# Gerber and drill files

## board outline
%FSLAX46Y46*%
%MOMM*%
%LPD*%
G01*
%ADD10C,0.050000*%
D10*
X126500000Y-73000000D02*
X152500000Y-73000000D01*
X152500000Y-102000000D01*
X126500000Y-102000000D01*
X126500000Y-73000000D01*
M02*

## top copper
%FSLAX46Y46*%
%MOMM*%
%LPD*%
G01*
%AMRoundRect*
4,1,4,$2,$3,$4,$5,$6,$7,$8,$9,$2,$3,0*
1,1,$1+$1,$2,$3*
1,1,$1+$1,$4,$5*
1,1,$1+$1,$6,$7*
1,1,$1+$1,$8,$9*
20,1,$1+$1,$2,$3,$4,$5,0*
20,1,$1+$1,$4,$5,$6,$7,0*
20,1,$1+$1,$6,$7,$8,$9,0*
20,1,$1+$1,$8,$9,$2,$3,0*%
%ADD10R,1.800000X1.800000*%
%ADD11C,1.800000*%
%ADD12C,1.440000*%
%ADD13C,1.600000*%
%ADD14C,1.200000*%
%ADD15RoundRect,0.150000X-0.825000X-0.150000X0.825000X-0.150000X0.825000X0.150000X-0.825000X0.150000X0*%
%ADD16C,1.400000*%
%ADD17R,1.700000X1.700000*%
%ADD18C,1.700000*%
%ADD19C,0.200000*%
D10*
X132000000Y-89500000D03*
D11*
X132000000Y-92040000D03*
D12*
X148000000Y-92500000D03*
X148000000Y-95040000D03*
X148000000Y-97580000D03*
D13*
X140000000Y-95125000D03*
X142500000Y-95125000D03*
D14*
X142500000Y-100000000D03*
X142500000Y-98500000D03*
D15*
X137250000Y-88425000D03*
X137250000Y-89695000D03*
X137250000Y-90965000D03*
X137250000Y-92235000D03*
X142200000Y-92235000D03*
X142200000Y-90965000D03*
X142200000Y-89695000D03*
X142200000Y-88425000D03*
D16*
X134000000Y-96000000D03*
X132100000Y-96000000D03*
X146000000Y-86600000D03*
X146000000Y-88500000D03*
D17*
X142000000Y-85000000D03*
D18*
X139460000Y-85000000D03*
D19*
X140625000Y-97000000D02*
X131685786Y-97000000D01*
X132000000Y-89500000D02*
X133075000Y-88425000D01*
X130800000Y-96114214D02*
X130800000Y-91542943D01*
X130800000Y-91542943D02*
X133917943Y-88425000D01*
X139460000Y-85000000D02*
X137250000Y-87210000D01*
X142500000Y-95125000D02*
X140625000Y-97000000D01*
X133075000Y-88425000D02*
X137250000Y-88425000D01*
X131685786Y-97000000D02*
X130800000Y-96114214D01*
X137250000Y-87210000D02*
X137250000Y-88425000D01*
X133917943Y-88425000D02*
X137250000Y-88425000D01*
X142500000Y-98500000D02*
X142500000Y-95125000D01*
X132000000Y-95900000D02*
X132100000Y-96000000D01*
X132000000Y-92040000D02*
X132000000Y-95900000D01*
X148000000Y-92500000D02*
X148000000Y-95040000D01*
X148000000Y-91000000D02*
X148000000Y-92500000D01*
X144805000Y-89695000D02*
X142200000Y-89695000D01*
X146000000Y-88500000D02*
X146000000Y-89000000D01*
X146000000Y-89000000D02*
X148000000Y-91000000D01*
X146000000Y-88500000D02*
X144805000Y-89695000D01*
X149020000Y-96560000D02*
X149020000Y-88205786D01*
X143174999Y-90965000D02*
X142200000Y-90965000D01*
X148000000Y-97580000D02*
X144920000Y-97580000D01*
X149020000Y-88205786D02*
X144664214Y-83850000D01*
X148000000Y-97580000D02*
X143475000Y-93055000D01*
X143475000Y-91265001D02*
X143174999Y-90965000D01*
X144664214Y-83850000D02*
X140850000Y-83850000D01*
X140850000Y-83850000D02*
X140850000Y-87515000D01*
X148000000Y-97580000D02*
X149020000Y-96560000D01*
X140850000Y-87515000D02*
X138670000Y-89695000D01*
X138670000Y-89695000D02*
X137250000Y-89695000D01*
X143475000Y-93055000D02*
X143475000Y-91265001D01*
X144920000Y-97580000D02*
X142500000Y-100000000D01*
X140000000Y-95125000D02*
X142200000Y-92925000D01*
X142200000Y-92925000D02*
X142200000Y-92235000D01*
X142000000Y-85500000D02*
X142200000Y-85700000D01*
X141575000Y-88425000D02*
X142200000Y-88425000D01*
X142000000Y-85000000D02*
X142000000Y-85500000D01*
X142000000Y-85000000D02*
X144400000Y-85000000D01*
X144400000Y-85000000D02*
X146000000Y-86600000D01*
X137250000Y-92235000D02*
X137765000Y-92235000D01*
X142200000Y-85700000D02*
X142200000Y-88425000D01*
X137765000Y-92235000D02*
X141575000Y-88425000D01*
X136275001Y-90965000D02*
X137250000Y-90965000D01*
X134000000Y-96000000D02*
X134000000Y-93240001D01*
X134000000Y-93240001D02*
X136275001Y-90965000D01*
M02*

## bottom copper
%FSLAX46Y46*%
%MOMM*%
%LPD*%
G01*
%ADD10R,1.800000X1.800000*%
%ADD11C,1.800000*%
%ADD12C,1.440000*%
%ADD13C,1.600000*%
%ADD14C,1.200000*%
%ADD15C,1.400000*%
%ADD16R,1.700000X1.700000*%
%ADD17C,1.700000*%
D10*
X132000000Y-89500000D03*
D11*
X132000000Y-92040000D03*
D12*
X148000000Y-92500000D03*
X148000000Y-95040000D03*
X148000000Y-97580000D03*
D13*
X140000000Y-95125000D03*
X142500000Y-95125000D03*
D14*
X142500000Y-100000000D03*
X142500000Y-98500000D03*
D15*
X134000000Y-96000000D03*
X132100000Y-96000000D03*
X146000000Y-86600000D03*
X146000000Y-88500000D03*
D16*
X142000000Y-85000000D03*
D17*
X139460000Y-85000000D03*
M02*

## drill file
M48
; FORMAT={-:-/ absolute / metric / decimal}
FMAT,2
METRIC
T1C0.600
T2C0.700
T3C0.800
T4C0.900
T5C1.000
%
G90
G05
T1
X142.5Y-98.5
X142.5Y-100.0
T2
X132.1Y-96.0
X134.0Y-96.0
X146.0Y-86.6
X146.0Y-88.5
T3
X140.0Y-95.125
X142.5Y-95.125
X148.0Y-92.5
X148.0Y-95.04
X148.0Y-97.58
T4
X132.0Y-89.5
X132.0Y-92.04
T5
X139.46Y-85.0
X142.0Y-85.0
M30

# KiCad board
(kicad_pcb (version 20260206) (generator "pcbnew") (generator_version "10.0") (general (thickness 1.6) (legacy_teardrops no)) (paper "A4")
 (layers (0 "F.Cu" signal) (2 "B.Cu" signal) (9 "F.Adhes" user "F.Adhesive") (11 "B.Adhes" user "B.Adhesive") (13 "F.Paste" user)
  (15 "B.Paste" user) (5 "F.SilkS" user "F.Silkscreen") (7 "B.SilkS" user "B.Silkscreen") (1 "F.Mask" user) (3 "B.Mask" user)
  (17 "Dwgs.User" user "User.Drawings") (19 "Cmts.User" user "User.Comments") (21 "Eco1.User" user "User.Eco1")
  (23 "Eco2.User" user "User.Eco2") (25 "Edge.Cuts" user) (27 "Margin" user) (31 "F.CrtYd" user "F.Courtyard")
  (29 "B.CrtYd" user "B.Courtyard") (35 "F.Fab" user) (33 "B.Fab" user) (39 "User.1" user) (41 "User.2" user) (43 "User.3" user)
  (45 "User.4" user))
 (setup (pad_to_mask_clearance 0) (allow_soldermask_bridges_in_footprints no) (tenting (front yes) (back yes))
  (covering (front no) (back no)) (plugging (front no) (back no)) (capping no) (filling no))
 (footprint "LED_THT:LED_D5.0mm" (layer "F.Cu") (at 132 89.5 -90)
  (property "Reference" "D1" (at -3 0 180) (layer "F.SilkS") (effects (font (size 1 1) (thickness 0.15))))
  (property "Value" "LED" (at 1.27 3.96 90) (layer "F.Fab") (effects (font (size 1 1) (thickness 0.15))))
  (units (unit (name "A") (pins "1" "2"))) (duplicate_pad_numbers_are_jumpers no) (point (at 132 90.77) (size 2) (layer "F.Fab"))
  (pad "1" thru_hole rect (at 0 0 270) (size 1.8 1.8) (drill 0.9) (layers "*.Cu" "*.Mask") (remove_unused_layers no) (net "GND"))
  (pad "2" thru_hole circle (at 2.54 0 270) (size 1.8 1.8) (drill 0.9) (layers "*.Cu" "*.Mask") (remove_unused_layers no) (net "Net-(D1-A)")))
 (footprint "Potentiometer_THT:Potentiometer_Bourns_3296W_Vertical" (layer "F.Cu") (at 148 92.5 90)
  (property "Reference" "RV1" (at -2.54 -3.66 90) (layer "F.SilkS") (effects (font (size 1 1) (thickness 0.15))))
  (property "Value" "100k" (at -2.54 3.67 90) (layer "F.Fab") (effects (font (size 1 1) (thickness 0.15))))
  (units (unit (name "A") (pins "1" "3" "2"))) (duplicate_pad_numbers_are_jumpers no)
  (pad "1" thru_hole circle (at 0 0 90) (size 1.44 1.44) (drill 0.8) (layers "*.Cu" "*.Mask") (remove_unused_layers no)
   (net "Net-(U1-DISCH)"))
  (pad "2" thru_hole circle (at -2.54 0 90) (size 1.44 1.44) (drill 0.8) (layers "*.Cu" "*.Mask") (remove_unused_layers no)
   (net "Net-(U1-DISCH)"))
  (pad "3" thru_hole circle (at -5.08 0 90) (size 1.44 1.44) (drill 0.8) (layers "*.Cu" "*.Mask") (remove_unused_layers no)
   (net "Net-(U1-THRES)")))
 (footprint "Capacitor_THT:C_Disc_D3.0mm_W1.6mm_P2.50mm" (layer "F.Cu") (at 140 95.125)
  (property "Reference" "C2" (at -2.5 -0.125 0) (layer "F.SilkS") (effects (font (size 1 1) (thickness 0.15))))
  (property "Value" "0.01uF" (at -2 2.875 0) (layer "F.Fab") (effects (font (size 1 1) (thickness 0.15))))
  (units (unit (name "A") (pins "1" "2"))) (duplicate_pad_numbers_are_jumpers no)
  (pad "1" thru_hole circle (at 0 0) (size 1.6 1.6) (drill 0.8) (layers "*.Cu" "*.Mask") (remove_unused_layers no) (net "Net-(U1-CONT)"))
  (pad "2" thru_hole circle (at 2.5 0) (size 1.6 1.6) (drill 0.8) (layers "*.Cu" "*.Mask") (remove_unused_layers no) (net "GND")))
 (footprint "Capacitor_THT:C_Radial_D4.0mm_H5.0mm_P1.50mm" (layer "F.Cu") (at 142.5 100 90)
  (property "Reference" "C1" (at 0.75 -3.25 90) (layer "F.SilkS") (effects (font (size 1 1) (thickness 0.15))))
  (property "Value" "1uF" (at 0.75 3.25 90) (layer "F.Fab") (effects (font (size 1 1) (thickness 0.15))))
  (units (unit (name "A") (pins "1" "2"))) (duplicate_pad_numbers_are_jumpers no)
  (pad "1" thru_hole circle (at 0 0 90) (size 1.2 1.2) (drill 0.6) (layers "*.Cu" "*.Mask") (remove_unused_layers no) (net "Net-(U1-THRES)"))
  (pad "2" thru_hole circle (at 1.5 0 90) (size 1.2 1.2) (drill 0.6) (layers "*.Cu" "*.Mask") (remove_unused_layers no) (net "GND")))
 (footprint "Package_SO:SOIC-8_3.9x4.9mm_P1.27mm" (layer "F.Cu") (at 139.725 90.33)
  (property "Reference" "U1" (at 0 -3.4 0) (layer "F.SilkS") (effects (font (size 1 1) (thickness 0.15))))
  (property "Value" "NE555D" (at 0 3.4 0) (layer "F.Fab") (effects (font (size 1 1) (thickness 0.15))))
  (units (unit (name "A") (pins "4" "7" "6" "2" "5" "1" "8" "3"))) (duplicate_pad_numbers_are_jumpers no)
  (pad "1" smd roundrect (at -2.475 -1.905) (size 1.95 0.6) (layers "F.Cu" "F.Mask" "F.Paste") (roundrect_rratio 0.25) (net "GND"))
  (pad "2" smd roundrect (at -2.475 -0.635) (size 1.95 0.6) (layers "F.Cu" "F.Mask" "F.Paste") (roundrect_rratio 0.25)
   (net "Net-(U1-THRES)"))
  (pad "3" smd roundrect (at -2.475 0.635) (size 1.95 0.6) (layers "F.Cu" "F.Mask" "F.Paste") (roundrect_rratio 0.25) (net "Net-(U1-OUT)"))
  (pad "4" smd roundrect (at -2.475 1.905) (size 1.95 0.6) (layers "F.Cu" "F.Mask" "F.Paste") (roundrect_rratio 0.25) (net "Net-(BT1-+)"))
  (pad "5" smd roundrect (at 2.475 1.905) (size 1.95 0.6) (layers "F.Cu" "F.Mask" "F.Paste") (roundrect_rratio 0.25) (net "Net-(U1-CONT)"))
  (pad "6" smd roundrect (at 2.475 0.635) (size 1.95 0.6) (layers "F.Cu" "F.Mask" "F.Paste") (roundrect_rratio 0.25) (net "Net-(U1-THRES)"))
  (pad "7" smd roundrect (at 2.475 -0.635) (size 1.95 0.6) (layers "F.Cu" "F.Mask" "F.Paste") (roundrect_rratio 0.25) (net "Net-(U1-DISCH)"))
  (pad "8" smd roundrect (at 2.475 -1.905) (size 1.95 0.6) (layers "F.Cu" "F.Mask" "F.Paste") (roundrect_rratio 0.25) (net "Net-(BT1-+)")))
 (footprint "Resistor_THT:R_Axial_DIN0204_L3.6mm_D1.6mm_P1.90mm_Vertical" (layer "F.Cu") (at 134 96 180)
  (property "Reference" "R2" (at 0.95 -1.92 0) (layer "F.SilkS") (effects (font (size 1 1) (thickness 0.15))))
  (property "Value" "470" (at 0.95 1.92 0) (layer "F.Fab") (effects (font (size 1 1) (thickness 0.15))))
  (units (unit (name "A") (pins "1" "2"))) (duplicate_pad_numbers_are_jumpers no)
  (pad "1" thru_hole circle (at 0 0 180) (size 1.4 1.4) (drill 0.7) (layers "*.Cu" "*.Mask") (remove_unused_layers no) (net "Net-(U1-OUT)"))
  (pad "2" thru_hole circle (at 1.9 0 180) (size 1.4 1.4) (drill 0.7) (layers "*.Cu" "*.Mask") (remove_unused_layers no) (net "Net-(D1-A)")))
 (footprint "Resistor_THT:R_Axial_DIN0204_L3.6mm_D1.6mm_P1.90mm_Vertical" (layer "F.Cu") (at 146 86.6 -90)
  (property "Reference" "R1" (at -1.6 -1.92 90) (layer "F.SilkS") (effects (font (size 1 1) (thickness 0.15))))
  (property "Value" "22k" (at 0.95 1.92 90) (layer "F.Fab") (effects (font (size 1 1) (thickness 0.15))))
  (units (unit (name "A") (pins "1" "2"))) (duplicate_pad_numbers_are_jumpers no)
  (pad "1" thru_hole circle (at 0 0 270) (size 1.4 1.4) (drill 0.7) (layers "*.Cu" "*.Mask") (remove_unused_layers no) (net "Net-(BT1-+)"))
  (pad "2" thru_hole circle (at 1.9 0 270) (size 1.4 1.4) (drill 0.7) (layers "*.Cu" "*.Mask") (remove_unused_layers no)
   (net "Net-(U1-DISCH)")))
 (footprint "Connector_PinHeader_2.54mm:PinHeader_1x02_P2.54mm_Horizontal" (layer "B.Cu") (at 142 85 90)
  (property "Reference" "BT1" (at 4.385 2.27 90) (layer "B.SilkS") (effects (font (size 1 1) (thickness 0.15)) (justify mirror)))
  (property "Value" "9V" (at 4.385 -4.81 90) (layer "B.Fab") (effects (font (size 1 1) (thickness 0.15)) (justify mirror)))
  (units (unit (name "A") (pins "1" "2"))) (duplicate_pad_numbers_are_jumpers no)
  (pad "1" thru_hole rect (at 0 0 90) (size 1.7 1.7) (drill 1) (layers "*.Cu" "*.Mask") (remove_unused_layers no) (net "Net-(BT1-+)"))
  (pad "2" thru_hole circle (at 0 -2.54 90) (size 1.7 1.7) (drill 1) (layers "*.Cu" "*.Mask") (remove_unused_layers no) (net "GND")))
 (gr_rect (start 126.5 73) (end 152.5 102) (stroke (width 0.05) (type default)) (fill no) (layer "Edge.Cuts"))
 (segment (start 140.625 97) (end 131.685786 97) (width 0.2) (layer "F.Cu") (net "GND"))
 (segment (start 132 89.5) (end 133.075 88.425) (width 0.2) (layer "F.Cu") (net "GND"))
 (segment (start 130.8 96.114214) (end 130.8 91.542943) (width 0.2) (layer "F.Cu") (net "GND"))
 (segment (start 130.8 91.542943) (end 133.917943 88.425) (width 0.2) (layer "F.Cu") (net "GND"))
 (segment (start 139.46 85) (end 137.25 87.21) (width 0.2) (layer "F.Cu") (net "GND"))
 (segment (start 142.5 95.125) (end 140.625 97) (width 0.2) (layer "F.Cu") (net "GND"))
 (segment (start 133.075 88.425) (end 137.25 88.425) (width 0.2) (layer "F.Cu") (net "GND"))
 (segment (start 131.685786 97) (end 130.8 96.114214) (width 0.2) (layer "F.Cu") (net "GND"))
 (segment (start 137.25 87.21) (end 137.25 88.425) (width 0.2) (layer "F.Cu") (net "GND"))
 (segment (start 133.917943 88.425) (end 137.25 88.425) (width 0.2) (layer "F.Cu") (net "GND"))
 (segment (start 142.5 98.5) (end 142.5 95.125) (width 0.2) (layer "F.Cu") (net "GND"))
 (segment (start 132 95.9) (end 132.1 96) (width 0.2) (layer "F.Cu") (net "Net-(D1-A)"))
 (segment (start 132 92.04) (end 132 95.9) (width 0.2) (layer "F.Cu") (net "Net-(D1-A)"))
 (segment (start 148 92.5) (end 148 95.04) (width 0.2) (layer "F.Cu") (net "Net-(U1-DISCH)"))
 (segment (start 148 91) (end 148 92.5) (width 0.2) (layer "F.Cu") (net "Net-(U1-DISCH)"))
 (segment (start 144.805 89.695) (end 142.2 89.695) (width 0.2) (layer "F.Cu") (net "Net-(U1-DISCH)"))
 (segment (start 146 88.5) (end 146 89) (width 0.2) (layer "F.Cu") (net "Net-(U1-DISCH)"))
 (segment (start 146 89) (end 148 91) (width 0.2) (layer "F.Cu") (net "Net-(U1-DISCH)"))
 (segment (start 146 88.5) (end 144.805 89.695) (width 0.2) (layer "F.Cu") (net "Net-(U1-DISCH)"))
 (segment (start 149.02 96.56) (end 149.02 88.205786) (width 0.2) (layer "F.Cu") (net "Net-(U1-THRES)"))
 (segment (start 143.174999 90.965) (end 142.2 90.965) (width 0.2) (layer "F.Cu") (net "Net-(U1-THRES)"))
 (segment (start 148 97.58) (end 144.92 97.58) (width 0.2) (layer "F.Cu") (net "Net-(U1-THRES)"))
 (segment (start 149.02 88.205786) (end 144.664214 83.85) (width 0.2) (layer "F.Cu") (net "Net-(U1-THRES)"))
 (segment (start 148 97.58) (end 143.475 93.055) (width 0.2) (layer "F.Cu") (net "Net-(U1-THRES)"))
 (segment (start 143.475 91.265001) (end 143.174999 90.965) (width 0.2) (layer "F.Cu") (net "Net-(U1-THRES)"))
 (segment (start 144.664214 83.85) (end 140.85 83.85) (width 0.2) (layer "F.Cu") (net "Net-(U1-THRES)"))
 (segment (start 140.85 83.85) (end 140.85 87.515) (width 0.2) (layer "F.Cu") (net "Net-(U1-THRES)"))
 (segment (start 148 97.58) (end 149.02 96.56) (width 0.2) (layer "F.Cu") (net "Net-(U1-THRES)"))
 (segment (start 140.85 87.515) (end 138.67 89.695) (width 0.2) (layer "F.Cu") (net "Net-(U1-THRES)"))
 (segment (start 138.67 89.695) (end 137.25 89.695) (width 0.2) (layer "F.Cu") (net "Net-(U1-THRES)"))
 (segment (start 143.475 93.055) (end 143.475 91.265001) (width 0.2) (layer "F.Cu") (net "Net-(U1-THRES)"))
 (segment (start 144.92 97.58) (end 142.5 100) (width 0.2) (layer "F.Cu") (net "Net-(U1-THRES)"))
 (segment (start 140 95.125) (end 142.2 92.925) (width 0.2) (layer "F.Cu") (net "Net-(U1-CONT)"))
 (segment (start 142.2 92.925) (end 142.2 92.235) (width 0.2) (layer "F.Cu") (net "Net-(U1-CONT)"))
 (segment (start 142 85.5) (end 142.2 85.7) (width 0.2) (layer "F.Cu") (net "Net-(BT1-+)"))
 (segment (start 141.575 88.425) (end 142.2 88.425) (width 0.2) (layer "F.Cu") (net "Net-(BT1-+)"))
 (segment (start 142 85) (end 142 85.5) (width 0.2) (layer "F.Cu") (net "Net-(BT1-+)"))
 (segment (start 142 85) (end 144.4 85) (width 0.2) (layer "F.Cu") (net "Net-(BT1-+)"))
 (segment (start 144.4 85) (end 146 86.6) (width 0.2) (layer "F.Cu") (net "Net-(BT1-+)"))
 (segment (start 137.25 92.235) (end 137.765 92.235) (width 0.2) (layer "F.Cu") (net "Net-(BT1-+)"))
 (segment (start 142.2 85.7) (end 142.2 88.425) (width 0.2) (layer "F.Cu") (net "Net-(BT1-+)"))
 (segment (start 137.765 92.235) (end 141.575 88.425) (width 0.2) (layer "F.Cu") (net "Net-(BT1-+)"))
 (segment (start 136.275001 90.965) (end 137.25 90.965) (width 0.2) (layer "F.Cu") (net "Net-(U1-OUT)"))
 (segment (start 134 96) (end 134 93.240001) (width 0.2) (layer "F.Cu") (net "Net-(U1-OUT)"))
 (segment (start 134 93.240001) (end 136.275001 90.965) (width 0.2) (layer "F.Cu") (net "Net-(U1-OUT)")))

